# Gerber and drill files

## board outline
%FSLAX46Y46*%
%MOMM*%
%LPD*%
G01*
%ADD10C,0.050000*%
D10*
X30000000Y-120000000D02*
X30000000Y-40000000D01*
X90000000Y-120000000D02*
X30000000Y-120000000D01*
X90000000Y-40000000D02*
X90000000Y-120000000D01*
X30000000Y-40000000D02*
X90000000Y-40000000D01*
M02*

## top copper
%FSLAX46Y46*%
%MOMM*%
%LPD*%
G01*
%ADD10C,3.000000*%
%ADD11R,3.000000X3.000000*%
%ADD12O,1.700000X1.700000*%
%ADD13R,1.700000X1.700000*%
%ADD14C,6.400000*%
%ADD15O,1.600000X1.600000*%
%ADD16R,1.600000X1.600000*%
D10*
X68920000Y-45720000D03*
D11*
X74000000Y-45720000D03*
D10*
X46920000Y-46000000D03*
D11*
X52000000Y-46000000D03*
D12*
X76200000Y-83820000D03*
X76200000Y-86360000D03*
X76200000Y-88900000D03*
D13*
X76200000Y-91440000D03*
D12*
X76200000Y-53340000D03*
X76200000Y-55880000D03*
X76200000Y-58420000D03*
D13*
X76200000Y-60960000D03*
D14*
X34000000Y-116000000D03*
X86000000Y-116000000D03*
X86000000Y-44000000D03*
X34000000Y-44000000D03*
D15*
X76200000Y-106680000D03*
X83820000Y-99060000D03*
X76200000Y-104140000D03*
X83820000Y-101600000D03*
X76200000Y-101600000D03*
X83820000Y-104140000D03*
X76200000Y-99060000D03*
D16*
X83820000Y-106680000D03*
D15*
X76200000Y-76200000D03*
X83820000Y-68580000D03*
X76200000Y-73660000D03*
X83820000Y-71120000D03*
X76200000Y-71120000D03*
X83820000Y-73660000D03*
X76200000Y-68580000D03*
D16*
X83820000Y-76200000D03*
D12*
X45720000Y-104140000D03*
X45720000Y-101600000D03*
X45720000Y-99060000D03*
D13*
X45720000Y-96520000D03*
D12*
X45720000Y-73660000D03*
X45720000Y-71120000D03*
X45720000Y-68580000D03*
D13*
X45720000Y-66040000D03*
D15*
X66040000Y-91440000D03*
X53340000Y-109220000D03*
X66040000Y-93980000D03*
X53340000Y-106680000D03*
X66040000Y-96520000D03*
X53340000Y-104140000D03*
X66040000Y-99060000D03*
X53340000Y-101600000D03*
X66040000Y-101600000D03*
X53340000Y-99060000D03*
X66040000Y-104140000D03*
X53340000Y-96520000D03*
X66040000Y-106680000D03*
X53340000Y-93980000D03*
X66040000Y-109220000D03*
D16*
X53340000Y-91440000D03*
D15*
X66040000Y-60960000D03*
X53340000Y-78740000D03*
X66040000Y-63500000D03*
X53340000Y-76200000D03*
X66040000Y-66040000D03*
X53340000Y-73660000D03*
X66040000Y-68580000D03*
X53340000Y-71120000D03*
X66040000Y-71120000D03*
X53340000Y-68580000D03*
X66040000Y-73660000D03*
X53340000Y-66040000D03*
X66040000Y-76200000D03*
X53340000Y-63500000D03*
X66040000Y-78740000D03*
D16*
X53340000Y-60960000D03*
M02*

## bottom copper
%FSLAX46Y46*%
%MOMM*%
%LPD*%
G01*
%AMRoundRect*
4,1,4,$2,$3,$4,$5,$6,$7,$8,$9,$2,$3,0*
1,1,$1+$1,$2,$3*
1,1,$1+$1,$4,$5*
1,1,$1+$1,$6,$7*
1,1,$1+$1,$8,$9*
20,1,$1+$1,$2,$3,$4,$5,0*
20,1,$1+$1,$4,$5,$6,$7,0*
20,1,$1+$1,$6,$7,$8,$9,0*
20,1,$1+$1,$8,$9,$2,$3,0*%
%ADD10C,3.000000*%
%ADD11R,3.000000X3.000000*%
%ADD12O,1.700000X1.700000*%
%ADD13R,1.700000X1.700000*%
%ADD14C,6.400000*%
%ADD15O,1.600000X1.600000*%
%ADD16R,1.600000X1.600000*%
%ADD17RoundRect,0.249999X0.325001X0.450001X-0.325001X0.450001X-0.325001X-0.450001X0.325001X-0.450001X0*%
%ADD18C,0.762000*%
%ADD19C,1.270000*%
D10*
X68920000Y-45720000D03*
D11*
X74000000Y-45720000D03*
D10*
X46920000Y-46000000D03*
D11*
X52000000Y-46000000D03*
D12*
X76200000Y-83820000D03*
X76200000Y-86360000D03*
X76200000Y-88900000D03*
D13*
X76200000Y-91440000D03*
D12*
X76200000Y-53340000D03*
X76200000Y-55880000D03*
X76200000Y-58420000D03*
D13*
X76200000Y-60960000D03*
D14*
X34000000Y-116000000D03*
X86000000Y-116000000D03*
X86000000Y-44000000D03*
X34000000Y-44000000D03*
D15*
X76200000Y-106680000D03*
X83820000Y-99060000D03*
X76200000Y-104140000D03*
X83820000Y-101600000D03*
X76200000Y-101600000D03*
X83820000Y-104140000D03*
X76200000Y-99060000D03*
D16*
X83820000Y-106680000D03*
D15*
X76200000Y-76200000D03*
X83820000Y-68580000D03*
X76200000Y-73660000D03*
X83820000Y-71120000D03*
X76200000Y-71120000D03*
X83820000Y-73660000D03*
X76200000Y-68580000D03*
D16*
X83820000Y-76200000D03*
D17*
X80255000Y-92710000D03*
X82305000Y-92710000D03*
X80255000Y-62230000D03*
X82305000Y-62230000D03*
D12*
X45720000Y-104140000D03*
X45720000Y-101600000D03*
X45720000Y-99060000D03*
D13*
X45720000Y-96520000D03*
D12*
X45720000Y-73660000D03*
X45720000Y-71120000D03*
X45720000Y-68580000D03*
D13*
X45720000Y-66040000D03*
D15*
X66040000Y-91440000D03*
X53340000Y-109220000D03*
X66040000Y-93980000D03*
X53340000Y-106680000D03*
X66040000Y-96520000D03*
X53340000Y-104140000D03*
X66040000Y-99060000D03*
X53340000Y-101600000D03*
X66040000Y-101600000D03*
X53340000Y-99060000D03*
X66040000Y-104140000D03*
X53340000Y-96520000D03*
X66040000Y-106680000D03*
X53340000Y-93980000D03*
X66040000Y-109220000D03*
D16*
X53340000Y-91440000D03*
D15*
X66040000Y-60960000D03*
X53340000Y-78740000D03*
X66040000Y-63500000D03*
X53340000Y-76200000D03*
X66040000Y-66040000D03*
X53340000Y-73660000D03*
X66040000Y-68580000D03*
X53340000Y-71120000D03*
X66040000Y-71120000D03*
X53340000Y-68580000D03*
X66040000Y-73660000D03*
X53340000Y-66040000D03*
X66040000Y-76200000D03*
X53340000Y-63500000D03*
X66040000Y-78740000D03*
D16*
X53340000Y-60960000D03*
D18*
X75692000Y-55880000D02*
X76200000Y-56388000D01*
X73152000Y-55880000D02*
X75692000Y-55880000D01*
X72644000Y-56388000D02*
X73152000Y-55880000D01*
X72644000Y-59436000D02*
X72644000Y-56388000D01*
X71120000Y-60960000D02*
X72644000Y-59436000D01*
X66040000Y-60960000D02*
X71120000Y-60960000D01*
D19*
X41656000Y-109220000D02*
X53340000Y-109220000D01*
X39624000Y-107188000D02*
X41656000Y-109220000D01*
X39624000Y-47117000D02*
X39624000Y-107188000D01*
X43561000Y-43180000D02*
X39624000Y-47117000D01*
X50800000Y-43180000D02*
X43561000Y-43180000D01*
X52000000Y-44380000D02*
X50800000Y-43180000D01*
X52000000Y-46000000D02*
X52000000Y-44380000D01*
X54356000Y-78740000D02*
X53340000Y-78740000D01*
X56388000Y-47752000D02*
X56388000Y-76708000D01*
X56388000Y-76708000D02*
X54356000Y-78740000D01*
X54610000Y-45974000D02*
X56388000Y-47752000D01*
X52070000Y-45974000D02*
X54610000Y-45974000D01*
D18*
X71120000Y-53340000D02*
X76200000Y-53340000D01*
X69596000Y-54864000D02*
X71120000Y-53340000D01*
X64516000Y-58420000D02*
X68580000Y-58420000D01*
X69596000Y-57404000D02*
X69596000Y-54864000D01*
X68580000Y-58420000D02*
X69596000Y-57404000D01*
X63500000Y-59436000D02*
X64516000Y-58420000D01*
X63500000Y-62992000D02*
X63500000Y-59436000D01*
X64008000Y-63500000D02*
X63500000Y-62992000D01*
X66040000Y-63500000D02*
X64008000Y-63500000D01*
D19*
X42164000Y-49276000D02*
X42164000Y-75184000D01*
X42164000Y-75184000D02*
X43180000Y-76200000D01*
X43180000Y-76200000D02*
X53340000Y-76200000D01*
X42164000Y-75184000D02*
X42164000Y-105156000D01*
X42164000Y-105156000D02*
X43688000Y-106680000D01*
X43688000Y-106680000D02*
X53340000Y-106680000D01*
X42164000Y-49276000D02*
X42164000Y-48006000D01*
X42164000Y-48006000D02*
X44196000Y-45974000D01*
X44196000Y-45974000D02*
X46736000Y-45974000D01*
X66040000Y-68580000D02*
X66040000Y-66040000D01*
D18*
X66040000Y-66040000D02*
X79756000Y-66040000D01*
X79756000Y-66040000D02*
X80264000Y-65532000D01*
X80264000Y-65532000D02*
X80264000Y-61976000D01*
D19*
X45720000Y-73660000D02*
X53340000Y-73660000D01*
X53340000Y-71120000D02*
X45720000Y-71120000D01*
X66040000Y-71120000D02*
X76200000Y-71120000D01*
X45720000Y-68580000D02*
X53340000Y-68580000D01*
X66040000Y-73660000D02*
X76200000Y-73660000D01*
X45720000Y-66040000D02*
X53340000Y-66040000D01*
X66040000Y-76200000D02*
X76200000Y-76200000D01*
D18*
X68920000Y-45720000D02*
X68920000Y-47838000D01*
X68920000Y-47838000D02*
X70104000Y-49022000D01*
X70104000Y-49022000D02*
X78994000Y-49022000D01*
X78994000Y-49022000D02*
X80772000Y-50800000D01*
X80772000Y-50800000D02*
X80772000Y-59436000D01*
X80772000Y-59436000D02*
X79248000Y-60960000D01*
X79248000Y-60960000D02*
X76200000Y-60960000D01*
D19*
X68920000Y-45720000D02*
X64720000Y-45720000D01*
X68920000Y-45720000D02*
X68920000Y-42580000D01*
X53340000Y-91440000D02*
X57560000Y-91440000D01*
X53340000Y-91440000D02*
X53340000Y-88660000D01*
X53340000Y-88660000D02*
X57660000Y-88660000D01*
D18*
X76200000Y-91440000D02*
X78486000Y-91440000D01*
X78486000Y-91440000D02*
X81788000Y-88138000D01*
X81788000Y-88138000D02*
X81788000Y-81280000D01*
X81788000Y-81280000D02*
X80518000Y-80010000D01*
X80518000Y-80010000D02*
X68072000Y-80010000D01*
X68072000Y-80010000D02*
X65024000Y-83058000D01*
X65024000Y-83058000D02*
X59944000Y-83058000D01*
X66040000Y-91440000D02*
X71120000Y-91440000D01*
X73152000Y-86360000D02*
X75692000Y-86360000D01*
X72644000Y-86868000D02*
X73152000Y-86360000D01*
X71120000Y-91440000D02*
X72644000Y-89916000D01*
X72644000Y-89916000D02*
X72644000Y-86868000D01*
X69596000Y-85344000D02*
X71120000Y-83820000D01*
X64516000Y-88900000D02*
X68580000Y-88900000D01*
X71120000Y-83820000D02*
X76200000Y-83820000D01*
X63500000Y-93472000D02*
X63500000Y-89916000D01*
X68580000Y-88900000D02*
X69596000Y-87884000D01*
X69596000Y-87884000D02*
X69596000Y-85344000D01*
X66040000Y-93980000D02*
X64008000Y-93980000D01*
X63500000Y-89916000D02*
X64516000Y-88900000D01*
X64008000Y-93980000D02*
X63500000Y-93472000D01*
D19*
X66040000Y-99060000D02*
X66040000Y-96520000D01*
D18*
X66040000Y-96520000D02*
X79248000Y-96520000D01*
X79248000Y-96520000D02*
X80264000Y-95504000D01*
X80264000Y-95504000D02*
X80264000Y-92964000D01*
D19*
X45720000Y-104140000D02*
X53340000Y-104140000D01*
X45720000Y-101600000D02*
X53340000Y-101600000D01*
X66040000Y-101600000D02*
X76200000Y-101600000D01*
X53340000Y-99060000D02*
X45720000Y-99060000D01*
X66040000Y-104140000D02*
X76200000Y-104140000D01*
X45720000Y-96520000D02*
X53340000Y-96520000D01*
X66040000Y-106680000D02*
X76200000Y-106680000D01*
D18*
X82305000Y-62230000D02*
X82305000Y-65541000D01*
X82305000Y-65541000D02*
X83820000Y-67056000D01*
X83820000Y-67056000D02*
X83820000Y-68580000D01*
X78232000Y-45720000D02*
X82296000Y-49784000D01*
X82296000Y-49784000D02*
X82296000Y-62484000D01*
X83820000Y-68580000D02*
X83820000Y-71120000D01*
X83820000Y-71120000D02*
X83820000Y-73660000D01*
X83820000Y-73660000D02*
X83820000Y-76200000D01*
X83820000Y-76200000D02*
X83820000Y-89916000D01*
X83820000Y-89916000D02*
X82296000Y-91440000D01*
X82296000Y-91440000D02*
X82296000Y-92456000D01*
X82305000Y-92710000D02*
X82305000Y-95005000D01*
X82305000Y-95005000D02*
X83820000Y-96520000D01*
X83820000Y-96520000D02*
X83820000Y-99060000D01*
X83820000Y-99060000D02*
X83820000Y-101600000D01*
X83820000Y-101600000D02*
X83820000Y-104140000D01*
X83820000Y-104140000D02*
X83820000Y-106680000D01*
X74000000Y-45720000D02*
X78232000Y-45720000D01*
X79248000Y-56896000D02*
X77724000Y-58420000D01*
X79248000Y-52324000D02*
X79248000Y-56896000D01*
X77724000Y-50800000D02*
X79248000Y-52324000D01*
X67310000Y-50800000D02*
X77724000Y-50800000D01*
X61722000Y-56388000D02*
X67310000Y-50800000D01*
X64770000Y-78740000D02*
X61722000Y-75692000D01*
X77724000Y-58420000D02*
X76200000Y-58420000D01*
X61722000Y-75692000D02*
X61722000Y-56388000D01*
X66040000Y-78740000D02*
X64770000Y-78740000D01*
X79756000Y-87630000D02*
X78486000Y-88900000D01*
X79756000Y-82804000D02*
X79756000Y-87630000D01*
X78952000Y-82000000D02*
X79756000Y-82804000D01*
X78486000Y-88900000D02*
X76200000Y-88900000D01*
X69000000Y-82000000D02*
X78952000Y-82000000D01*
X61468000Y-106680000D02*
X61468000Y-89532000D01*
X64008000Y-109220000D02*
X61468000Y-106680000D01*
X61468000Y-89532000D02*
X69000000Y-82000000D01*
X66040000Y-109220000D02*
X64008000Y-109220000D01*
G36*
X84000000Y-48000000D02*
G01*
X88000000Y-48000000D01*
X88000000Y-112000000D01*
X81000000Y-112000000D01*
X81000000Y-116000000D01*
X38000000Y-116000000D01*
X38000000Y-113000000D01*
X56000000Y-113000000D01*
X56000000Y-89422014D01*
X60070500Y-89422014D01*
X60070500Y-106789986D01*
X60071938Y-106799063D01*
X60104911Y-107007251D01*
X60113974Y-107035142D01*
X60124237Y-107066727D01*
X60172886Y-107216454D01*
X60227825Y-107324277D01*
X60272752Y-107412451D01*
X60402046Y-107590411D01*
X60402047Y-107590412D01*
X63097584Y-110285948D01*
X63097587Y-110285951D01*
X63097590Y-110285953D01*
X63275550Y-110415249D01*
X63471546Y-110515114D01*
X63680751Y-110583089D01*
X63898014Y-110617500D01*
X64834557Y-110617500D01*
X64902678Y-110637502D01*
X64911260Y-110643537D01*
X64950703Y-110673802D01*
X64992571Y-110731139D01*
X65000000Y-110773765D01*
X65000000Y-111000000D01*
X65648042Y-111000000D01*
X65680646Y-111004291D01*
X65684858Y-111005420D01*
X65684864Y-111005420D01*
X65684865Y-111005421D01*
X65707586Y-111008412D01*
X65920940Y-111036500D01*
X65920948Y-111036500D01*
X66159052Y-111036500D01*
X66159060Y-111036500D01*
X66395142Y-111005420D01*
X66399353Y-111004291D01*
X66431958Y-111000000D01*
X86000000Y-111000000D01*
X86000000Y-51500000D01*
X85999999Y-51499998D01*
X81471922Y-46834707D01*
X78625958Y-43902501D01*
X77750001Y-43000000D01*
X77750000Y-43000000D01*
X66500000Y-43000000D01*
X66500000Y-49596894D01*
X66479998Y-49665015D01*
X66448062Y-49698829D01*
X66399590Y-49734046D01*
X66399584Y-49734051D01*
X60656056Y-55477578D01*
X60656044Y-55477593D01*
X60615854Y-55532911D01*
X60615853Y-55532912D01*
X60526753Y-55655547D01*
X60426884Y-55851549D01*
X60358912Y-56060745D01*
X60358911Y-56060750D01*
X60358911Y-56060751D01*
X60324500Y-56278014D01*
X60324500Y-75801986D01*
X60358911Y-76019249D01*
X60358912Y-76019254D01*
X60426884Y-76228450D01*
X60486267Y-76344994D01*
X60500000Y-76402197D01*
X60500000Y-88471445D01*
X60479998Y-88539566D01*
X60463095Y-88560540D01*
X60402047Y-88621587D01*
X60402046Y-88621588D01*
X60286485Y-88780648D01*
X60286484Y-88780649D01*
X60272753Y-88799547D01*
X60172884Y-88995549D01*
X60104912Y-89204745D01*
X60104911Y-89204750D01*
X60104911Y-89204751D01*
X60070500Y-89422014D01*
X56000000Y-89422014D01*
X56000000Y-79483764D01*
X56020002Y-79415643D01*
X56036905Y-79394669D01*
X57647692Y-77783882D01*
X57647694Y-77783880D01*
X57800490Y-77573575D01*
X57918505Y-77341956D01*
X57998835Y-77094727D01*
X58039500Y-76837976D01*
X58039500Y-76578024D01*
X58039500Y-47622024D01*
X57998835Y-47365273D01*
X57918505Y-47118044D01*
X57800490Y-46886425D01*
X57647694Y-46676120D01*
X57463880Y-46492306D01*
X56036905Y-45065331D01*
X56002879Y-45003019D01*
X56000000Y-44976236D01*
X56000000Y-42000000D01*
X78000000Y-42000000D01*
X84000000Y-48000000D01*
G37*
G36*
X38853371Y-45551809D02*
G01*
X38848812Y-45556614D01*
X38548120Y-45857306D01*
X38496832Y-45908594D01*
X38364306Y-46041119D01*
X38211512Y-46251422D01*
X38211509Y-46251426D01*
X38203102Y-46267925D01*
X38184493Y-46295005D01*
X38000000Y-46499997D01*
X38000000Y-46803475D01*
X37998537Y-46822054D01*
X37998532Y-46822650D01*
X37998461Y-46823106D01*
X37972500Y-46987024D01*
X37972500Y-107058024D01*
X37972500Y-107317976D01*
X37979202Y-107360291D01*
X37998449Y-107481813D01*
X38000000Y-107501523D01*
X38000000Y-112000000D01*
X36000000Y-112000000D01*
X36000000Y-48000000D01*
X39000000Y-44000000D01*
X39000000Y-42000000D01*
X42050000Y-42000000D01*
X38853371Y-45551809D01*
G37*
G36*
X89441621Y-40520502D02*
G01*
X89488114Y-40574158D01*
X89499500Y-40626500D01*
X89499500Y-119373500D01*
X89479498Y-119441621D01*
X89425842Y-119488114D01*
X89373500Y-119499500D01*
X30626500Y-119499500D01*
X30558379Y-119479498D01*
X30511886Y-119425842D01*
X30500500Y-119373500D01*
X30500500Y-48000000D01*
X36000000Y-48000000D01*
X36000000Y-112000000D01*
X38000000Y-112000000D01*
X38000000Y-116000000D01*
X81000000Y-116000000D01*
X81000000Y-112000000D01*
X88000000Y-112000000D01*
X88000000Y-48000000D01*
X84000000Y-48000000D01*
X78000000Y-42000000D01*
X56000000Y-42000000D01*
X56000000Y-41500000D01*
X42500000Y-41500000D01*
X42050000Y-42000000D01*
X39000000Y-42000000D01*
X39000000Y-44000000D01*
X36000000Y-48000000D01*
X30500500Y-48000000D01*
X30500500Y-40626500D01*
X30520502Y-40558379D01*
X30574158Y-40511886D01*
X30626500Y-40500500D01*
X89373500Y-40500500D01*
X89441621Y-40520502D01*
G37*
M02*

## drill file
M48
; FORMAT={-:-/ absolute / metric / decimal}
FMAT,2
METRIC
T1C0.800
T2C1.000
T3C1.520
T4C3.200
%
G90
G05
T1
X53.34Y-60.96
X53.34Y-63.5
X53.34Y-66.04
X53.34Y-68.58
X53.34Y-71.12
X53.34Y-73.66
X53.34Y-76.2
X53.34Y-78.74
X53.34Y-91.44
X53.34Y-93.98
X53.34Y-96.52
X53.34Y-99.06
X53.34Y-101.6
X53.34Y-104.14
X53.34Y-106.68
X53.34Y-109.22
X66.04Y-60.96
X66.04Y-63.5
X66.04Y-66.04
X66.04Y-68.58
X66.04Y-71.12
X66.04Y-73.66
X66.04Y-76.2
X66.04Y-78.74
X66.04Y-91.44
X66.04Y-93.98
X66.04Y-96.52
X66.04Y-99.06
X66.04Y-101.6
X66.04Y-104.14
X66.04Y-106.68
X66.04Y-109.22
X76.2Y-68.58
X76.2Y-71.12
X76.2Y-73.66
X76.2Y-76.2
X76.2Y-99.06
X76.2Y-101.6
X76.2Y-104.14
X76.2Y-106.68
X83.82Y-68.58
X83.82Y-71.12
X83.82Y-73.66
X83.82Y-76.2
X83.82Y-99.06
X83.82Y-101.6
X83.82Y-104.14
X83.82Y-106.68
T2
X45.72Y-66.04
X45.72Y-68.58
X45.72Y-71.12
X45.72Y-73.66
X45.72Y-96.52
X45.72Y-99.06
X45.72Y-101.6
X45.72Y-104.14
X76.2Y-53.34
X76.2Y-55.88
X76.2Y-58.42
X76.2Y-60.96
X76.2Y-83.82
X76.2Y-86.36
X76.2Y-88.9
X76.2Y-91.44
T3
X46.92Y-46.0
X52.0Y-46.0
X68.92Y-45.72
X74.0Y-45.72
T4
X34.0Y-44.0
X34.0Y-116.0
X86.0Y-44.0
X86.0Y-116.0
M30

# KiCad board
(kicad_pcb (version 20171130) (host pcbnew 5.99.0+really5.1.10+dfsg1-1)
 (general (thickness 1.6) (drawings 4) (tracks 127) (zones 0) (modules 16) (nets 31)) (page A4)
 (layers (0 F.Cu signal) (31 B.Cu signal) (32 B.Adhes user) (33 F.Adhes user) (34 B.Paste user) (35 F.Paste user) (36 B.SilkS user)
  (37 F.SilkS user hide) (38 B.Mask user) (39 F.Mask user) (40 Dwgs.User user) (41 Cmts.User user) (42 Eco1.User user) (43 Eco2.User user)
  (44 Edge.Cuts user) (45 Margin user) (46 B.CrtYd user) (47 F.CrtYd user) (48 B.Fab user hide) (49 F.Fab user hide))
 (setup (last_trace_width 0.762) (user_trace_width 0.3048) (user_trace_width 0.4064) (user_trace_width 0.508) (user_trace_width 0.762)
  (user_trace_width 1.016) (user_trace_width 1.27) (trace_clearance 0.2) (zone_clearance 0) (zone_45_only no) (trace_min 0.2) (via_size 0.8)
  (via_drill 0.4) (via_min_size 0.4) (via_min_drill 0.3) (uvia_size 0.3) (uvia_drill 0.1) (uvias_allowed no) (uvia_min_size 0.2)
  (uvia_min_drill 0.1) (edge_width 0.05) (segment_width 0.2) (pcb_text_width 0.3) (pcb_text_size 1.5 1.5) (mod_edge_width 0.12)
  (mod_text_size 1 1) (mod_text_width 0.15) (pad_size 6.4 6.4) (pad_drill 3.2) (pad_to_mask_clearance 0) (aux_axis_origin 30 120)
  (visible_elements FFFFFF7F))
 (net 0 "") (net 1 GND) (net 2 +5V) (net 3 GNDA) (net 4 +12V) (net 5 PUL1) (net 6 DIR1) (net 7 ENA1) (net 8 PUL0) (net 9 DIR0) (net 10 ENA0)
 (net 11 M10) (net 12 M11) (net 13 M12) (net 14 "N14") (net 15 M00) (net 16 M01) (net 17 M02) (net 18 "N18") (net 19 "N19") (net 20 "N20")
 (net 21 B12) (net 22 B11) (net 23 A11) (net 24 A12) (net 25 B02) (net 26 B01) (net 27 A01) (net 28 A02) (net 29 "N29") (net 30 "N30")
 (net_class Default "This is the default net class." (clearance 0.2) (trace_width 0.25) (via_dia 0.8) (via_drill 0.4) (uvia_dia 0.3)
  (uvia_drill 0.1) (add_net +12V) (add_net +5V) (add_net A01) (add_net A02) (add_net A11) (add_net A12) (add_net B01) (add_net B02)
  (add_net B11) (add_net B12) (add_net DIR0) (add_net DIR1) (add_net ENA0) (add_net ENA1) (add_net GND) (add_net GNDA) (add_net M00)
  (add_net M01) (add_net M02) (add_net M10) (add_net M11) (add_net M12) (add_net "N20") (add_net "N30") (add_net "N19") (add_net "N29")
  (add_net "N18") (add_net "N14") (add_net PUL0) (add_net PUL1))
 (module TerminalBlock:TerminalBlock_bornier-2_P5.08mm (layer F.Cu) (at 74 45.72 180)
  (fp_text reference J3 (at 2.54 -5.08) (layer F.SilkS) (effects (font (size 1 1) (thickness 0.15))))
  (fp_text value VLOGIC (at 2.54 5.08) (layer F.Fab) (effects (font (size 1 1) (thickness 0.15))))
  (pad 2 thru_hole circle (at 5.08 0 180) (size 3 3) (drill 1.52) (layers *.Cu *.Mask) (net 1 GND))
  (pad 1 thru_hole rect (at 0 0 180) (size 3 3) (drill 1.52) (layers *.Cu *.Mask) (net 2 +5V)))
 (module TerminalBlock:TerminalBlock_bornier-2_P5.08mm (layer F.Cu) (at 52 46 180)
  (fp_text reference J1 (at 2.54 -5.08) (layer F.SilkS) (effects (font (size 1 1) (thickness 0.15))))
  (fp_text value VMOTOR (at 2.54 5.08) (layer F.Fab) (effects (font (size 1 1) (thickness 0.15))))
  (pad 2 thru_hole circle (at 5.08 0 180) (size 3 3) (drill 1.52) (layers *.Cu *.Mask) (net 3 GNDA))
  (pad 1 thru_hole rect (at 0 0 180) (size 3 3) (drill 1.52) (layers *.Cu *.Mask) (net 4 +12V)))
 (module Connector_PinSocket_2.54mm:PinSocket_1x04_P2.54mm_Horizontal (layer F.Cu) (at 76.2 91.44 180)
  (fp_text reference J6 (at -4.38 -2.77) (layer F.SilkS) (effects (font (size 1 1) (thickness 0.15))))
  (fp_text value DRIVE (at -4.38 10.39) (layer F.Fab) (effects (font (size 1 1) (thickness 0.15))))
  (pad 4 thru_hole oval (at 0 7.62 180) (size 1.7 1.7) (drill 1) (layers *.Cu *.Mask) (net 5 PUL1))
  (pad 3 thru_hole oval (at 0 5.08 180) (size 1.7 1.7) (drill 1) (layers *.Cu *.Mask) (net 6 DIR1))
  (pad 2 thru_hole oval (at 0 2.54 180) (size 1.7 1.7) (drill 1) (layers *.Cu *.Mask) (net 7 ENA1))
  (pad 1 thru_hole rect (at 0 0 180) (size 1.7 1.7) (drill 1) (layers *.Cu *.Mask) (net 1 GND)))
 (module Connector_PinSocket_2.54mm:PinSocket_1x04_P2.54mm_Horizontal (layer F.Cu) (at 76.2 60.96 180)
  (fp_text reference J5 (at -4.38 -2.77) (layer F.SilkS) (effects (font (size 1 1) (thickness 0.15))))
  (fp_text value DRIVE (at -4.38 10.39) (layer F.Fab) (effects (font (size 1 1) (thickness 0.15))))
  (pad 4 thru_hole oval (at 0 7.62 180) (size 1.7 1.7) (drill 1) (layers *.Cu *.Mask) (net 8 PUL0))
  (pad 3 thru_hole oval (at 0 5.08 180) (size 1.7 1.7) (drill 1) (layers *.Cu *.Mask) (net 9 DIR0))
  (pad 2 thru_hole oval (at 0 2.54 180) (size 1.7 1.7) (drill 1) (layers *.Cu *.Mask) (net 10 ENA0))
  (pad 1 thru_hole rect (at 0 0 180) (size 1.7 1.7) (drill 1) (layers *.Cu *.Mask) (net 1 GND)))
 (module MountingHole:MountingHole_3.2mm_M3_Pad (layer F.Cu) (at 34 116)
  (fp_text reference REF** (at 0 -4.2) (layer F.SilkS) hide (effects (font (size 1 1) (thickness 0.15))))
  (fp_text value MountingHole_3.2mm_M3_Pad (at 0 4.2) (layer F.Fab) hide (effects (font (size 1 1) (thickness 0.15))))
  (pad 1 thru_hole circle (at 0 0) (size 6.4 6.4) (drill 3.2) (layers *.Cu *.Mask) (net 1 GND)))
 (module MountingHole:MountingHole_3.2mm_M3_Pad (layer F.Cu) (at 86 116)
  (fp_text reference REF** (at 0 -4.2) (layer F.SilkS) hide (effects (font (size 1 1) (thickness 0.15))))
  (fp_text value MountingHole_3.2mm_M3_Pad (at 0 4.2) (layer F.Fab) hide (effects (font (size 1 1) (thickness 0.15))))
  (pad 1 thru_hole circle (at 0 0) (size 6.4 6.4) (drill 3.2) (layers *.Cu *.Mask) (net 1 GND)))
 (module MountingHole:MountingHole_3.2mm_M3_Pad (layer F.Cu) (at 86 44)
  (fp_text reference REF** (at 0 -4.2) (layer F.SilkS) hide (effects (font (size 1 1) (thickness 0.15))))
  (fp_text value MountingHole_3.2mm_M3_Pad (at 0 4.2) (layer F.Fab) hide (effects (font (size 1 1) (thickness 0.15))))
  (pad 1 thru_hole circle (at 0 0) (size 6.4 6.4) (drill 3.2) (layers *.Cu *.Mask) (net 1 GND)))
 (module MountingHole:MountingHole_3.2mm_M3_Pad (layer F.Cu) (at 34 44)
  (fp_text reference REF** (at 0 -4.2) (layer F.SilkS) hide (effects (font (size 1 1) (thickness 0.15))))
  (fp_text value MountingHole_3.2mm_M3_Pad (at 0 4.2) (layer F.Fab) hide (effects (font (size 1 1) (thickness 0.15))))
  (pad 1 thru_hole circle (at 0 0) (size 6.4 6.4) (drill 3.2) (layers *.Cu *.Mask) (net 1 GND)))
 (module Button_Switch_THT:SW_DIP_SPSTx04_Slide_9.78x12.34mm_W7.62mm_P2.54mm (layer F.Cu) (at 83.82 106.68 180)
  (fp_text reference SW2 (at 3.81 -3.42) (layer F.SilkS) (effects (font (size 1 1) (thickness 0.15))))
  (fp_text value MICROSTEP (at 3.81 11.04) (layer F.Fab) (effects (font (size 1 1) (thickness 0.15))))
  (pad 8 thru_hole oval (at 7.62 0 180) (size 1.6 1.6) (drill 0.8) (layers *.Cu *.Mask) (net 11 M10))
  (pad 4 thru_hole oval (at 0 7.62 180) (size 1.6 1.6) (drill 0.8) (layers *.Cu *.Mask) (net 2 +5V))
  (pad 7 thru_hole oval (at 7.62 2.54 180) (size 1.6 1.6) (drill 0.8) (layers *.Cu *.Mask) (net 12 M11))
  (pad 3 thru_hole oval (at 0 5.08 180) (size 1.6 1.6) (drill 0.8) (layers *.Cu *.Mask) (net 2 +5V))
  (pad 6 thru_hole oval (at 7.62 5.08 180) (size 1.6 1.6) (drill 0.8) (layers *.Cu *.Mask) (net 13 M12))
  (pad 2 thru_hole oval (at 0 2.54 180) (size 1.6 1.6) (drill 0.8) (layers *.Cu *.Mask) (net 2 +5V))
  (pad 5 thru_hole oval (at 7.62 7.62 180) (size 1.6 1.6) (drill 0.8) (layers *.Cu *.Mask) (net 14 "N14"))
  (pad 1 thru_hole rect (at 0 0 180) (size 1.6 1.6) (drill 0.8) (layers *.Cu *.Mask) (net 2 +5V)))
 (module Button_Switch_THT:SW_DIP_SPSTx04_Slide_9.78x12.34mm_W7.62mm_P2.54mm (layer F.Cu) (at 83.82 76.2 180)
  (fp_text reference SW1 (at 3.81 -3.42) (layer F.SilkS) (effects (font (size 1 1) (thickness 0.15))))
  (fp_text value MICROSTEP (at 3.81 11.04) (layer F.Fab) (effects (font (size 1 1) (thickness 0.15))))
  (pad 8 thru_hole oval (at 7.62 0 180) (size 1.6 1.6) (drill 0.8) (layers *.Cu *.Mask) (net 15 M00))
  (pad 4 thru_hole oval (at 0 7.62 180) (size 1.6 1.6) (drill 0.8) (layers *.Cu *.Mask) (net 2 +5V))
  (pad 7 thru_hole oval (at 7.62 2.54 180) (size 1.6 1.6) (drill 0.8) (layers *.Cu *.Mask) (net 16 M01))
  (pad 3 thru_hole oval (at 0 5.08 180) (size 1.6 1.6) (drill 0.8) (layers *.Cu *.Mask) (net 2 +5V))
  (pad 6 thru_hole oval (at 7.62 5.08 180) (size 1.6 1.6) (drill 0.8) (layers *.Cu *.Mask) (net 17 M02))
  (pad 2 thru_hole oval (at 0 2.54 180) (size 1.6 1.6) (drill 0.8) (layers *.Cu *.Mask) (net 2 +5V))
  (pad 5 thru_hole oval (at 7.62 7.62 180) (size 1.6 1.6) (drill 0.8) (layers *.Cu *.Mask) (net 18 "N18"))
  (pad 1 thru_hole rect (at 0 0 180) (size 1.6 1.6) (drill 0.8) (layers *.Cu *.Mask) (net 2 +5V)))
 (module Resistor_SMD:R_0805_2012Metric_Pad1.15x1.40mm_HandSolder (layer B.Cu) (at 81.28 92.71 180)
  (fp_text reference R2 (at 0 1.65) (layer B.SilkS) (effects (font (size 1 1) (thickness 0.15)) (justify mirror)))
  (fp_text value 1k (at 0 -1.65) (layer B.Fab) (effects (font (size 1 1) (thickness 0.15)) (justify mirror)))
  (pad 2 smd roundrect (at 1.025 0 180) (size 1.15 1.4) (layers B.Cu B.Paste B.Mask) (roundrect_rratio 0.2173904347826087) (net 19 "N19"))
  (pad 1 smd roundrect (at -1.025 0 180) (size 1.15 1.4) (layers B.Cu B.Paste B.Mask) (roundrect_rratio 0.2173904347826087) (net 2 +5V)))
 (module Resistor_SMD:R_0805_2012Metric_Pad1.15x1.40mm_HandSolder (layer B.Cu) (at 81.28 62.23 180)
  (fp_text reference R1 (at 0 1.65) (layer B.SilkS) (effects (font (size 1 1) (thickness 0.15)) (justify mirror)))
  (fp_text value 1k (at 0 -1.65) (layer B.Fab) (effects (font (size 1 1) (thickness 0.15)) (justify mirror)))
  (pad 2 smd roundrect (at 1.025 0 180) (size 1.15 1.4) (layers B.Cu B.Paste B.Mask) (roundrect_rratio 0.2173904347826087) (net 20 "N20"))
  (pad 1 smd roundrect (at -1.025 0 180) (size 1.15 1.4) (layers B.Cu B.Paste B.Mask) (roundrect_rratio 0.2173904347826087) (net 2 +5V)))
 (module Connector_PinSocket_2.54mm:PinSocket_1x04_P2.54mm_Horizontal (layer F.Cu) (at 45.72 96.52)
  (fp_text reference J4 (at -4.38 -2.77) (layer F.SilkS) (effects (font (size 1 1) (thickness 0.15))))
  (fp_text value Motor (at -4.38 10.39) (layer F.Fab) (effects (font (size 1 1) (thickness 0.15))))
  (pad 4 thru_hole oval (at 0 7.62) (size 1.7 1.7) (drill 1) (layers *.Cu *.Mask) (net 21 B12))
  (pad 3 thru_hole oval (at 0 5.08) (size 1.7 1.7) (drill 1) (layers *.Cu *.Mask) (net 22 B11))
  (pad 2 thru_hole oval (at 0 2.54) (size 1.7 1.7) (drill 1) (layers *.Cu *.Mask) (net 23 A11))
  (pad 1 thru_hole rect (at 0 0) (size 1.7 1.7) (drill 1) (layers *.Cu *.Mask) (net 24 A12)))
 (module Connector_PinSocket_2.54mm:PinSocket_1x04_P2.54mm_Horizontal (layer F.Cu) (at 45.72 66.04)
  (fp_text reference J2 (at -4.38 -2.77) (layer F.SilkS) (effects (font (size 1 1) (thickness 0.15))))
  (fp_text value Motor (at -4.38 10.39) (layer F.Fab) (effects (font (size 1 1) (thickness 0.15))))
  (pad 4 thru_hole oval (at 0 7.62) (size 1.7 1.7) (drill 1) (layers *.Cu *.Mask) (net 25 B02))
  (pad 3 thru_hole oval (at 0 5.08) (size 1.7 1.7) (drill 1) (layers *.Cu *.Mask) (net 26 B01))
  (pad 2 thru_hole oval (at 0 2.54) (size 1.7 1.7) (drill 1) (layers *.Cu *.Mask) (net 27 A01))
  (pad 1 thru_hole rect (at 0 0) (size 1.7 1.7) (drill 1) (layers *.Cu *.Mask) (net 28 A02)))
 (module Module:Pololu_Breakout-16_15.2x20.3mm (layer F.Cu) (at 53.34 91.44)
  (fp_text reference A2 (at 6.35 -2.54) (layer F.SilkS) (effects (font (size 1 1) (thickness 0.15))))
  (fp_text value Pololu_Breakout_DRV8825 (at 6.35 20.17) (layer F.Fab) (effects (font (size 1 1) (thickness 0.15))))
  (pad 16 thru_hole oval (at 12.7 0) (size 1.6 1.6) (drill 0.8) (layers *.Cu *.Mask) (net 6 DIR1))
  (pad 8 thru_hole oval (at 0 17.78) (size 1.6 1.6) (drill 0.8) (layers *.Cu *.Mask) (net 4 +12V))
  (pad 15 thru_hole oval (at 12.7 2.54) (size 1.6 1.6) (drill 0.8) (layers *.Cu *.Mask) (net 5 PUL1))
  (pad 7 thru_hole oval (at 0 15.24) (size 1.6 1.6) (drill 0.8) (layers *.Cu *.Mask) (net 3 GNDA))
  (pad 14 thru_hole oval (at 12.7 5.08) (size 1.6 1.6) (drill 0.8) (layers *.Cu *.Mask) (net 19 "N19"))
  (pad 6 thru_hole oval (at 0 12.7) (size 1.6 1.6) (drill 0.8) (layers *.Cu *.Mask) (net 21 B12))
  (pad 13 thru_hole oval (at 12.7 7.62) (size 1.6 1.6) (drill 0.8) (layers *.Cu *.Mask) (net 19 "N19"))
  (pad 5 thru_hole oval (at 0 10.16) (size 1.6 1.6) (drill 0.8) (layers *.Cu *.Mask) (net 22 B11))
  (pad 12 thru_hole oval (at 12.7 10.16) (size 1.6 1.6) (drill 0.8) (layers *.Cu *.Mask) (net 13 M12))
  (pad 4 thru_hole oval (at 0 7.62) (size 1.6 1.6) (drill 0.8) (layers *.Cu *.Mask) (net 23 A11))
  (pad 11 thru_hole oval (at 12.7 12.7) (size 1.6 1.6) (drill 0.8) (layers *.Cu *.Mask) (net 12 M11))
  (pad 3 thru_hole oval (at 0 5.08) (size 1.6 1.6) (drill 0.8) (layers *.Cu *.Mask) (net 24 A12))
  (pad 10 thru_hole oval (at 12.7 15.24) (size 1.6 1.6) (drill 0.8) (layers *.Cu *.Mask) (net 11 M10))
  (pad 2 thru_hole oval (at 0 2.54) (size 1.6 1.6) (drill 0.8) (layers *.Cu *.Mask) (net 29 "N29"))
  (pad 9 thru_hole oval (at 12.7 17.78) (size 1.6 1.6) (drill 0.8) (layers *.Cu *.Mask) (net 7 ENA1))
  (pad 1 thru_hole rect (at 0 0) (size 1.6 1.6) (drill 0.8) (layers *.Cu *.Mask) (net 1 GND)))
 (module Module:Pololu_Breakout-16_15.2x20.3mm (layer F.Cu) (at 53.34 60.96)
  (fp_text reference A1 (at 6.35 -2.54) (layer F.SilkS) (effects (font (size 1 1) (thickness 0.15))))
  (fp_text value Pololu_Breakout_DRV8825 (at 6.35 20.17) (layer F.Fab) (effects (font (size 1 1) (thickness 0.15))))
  (pad 16 thru_hole oval (at 12.7 0) (size 1.6 1.6) (drill 0.8) (layers *.Cu *.Mask) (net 9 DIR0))
  (pad 8 thru_hole oval (at 0 17.78) (size 1.6 1.6) (drill 0.8) (layers *.Cu *.Mask) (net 4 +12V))
  (pad 15 thru_hole oval (at 12.7 2.54) (size 1.6 1.6) (drill 0.8) (layers *.Cu *.Mask) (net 8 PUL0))
  (pad 7 thru_hole oval (at 0 15.24) (size 1.6 1.6) (drill 0.8) (layers *.Cu *.Mask) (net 3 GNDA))
  (pad 14 thru_hole oval (at 12.7 5.08) (size 1.6 1.6) (drill 0.8) (layers *.Cu *.Mask) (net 20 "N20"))
  (pad 6 thru_hole oval (at 0 12.7) (size 1.6 1.6) (drill 0.8) (layers *.Cu *.Mask) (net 25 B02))
  (pad 13 thru_hole oval (at 12.7 7.62) (size 1.6 1.6) (drill 0.8) (layers *.Cu *.Mask) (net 20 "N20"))
  (pad 5 thru_hole oval (at 0 10.16) (size 1.6 1.6) (drill 0.8) (layers *.Cu *.Mask) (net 26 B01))
  (pad 12 thru_hole oval (at 12.7 10.16) (size 1.6 1.6) (drill 0.8) (layers *.Cu *.Mask) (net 17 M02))
  (pad 4 thru_hole oval (at 0 7.62) (size 1.6 1.6) (drill 0.8) (layers *.Cu *.Mask) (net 27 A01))
  (pad 11 thru_hole oval (at 12.7 12.7) (size 1.6 1.6) (drill 0.8) (layers *.Cu *.Mask) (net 16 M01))
  (pad 3 thru_hole oval (at 0 5.08) (size 1.6 1.6) (drill 0.8) (layers *.Cu *.Mask) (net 28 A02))
  (pad 10 thru_hole oval (at 12.7 15.24) (size 1.6 1.6) (drill 0.8) (layers *.Cu *.Mask) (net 15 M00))
  (pad 2 thru_hole oval (at 0 2.54) (size 1.6 1.6) (drill 0.8) (layers *.Cu *.Mask) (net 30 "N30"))
  (pad 9 thru_hole oval (at 12.7 17.78) (size 1.6 1.6) (drill 0.8) (layers *.Cu *.Mask) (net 10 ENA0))
  (pad 1 thru_hole rect (at 0 0) (size 1.6 1.6) (drill 0.8) (layers *.Cu *.Mask) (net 1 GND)))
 (gr_line (start 30 120) (end 30 40) (layer Edge.Cuts) (width 0.05))
 (gr_line (start 90 120) (end 30 120) (layer Edge.Cuts) (width 0.05))
 (gr_line (start 90 40) (end 90 120) (layer Edge.Cuts) (width 0.05))
 (gr_line (start 30 40) (end 90 40) (layer Edge.Cuts) (width 0.05))
 (segment (start 75.692 55.88) (end 76.2 56.388) (width 0.762) (layer B.Cu) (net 9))
 (segment (start 73.152 55.88) (end 75.692 55.88) (width 0.762) (layer B.Cu) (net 9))
 (segment (start 72.644 56.388) (end 73.152 55.88) (width 0.762) (layer B.Cu) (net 9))
 (segment (start 72.644 59.436) (end 72.644 56.388) (width 0.762) (layer B.Cu) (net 9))
 (segment (start 71.12 60.96) (end 72.644 59.436) (width 0.762) (layer B.Cu) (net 9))
 (segment (start 66.04 60.96) (end 71.12 60.96) (width 0.762) (layer B.Cu) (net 9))
 (segment (start 41.656 109.22) (end 53.34 109.22) (width 1.27) (layer B.Cu) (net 4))
 (segment (start 39.624 107.188) (end 41.656 109.22) (width 1.27) (layer B.Cu) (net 4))
 (segment (start 39.624 47.117) (end 39.624 107.188) (width 1.27) (layer B.Cu) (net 4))
 (segment (start 43.561 43.18) (end 39.624 47.117) (width 1.27) (layer B.Cu) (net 4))
 (segment (start 50.8 43.18) (end 43.561 43.18) (width 1.27) (layer B.Cu) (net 4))
 (segment (start 52 44.38) (end 50.8 43.18) (width 1.27) (layer B.Cu) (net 4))
 (segment (start 52 46) (end 52 44.38) (width 1.27) (layer B.Cu) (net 4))
 (segment (start 54.356 78.74) (end 53.34 78.74) (width 1.27) (layer B.Cu) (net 4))
 (segment (start 56.388 47.752) (end 56.388 76.708) (width 1.27) (layer B.Cu) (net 4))
 (segment (start 56.388 76.708) (end 54.356 78.74) (width 1.27) (layer B.Cu) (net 4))
 (segment (start 54.61 45.974) (end 56.388 47.752) (width 1.27) (layer B.Cu) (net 4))
 (segment (start 52.07 45.974) (end 54.61 45.974) (width 1.27) (layer B.Cu) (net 4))
 (segment (start 71.12 53.34) (end 76.2 53.34) (width 0.762) (layer B.Cu) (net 8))
 (segment (start 69.596 54.864) (end 71.12 53.34) (width 0.762) (layer B.Cu) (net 8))
 (segment (start 64.516 58.42) (end 68.58 58.42) (width 0.762) (layer B.Cu) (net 8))
 (segment (start 69.596 57.404) (end 69.596 54.864) (width 0.762) (layer B.Cu) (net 8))
 (segment (start 68.58 58.42) (end 69.596 57.404) (width 0.762) (layer B.Cu) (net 8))
 (segment (start 63.5 59.436) (end 64.516 58.42) (width 0.762) (layer B.Cu) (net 8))
 (segment (start 63.5 62.992) (end 63.5 59.436) (width 0.762) (layer B.Cu) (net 8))
 (segment (start 64.008 63.5) (end 63.5 62.992) (width 0.762) (layer B.Cu) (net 8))
 (segment (start 66.04 63.5) (end 64.008 63.5) (width 0.762) (layer B.Cu) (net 8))
 (segment (start 42.164 49.276) (end 42.164 75.184) (width 1.27) (layer B.Cu) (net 3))
 (segment (start 42.164 75.184) (end 43.18 76.2) (width 1.27) (layer B.Cu) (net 3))
 (segment (start 43.18 76.2) (end 53.34 76.2) (width 1.27) (layer B.Cu) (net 3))
 (segment (start 42.164 75.184) (end 42.164 105.156) (width 1.27) (layer B.Cu) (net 3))
 (segment (start 42.164 105.156) (end 43.688 106.68) (width 1.27) (layer B.Cu) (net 3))
 (segment (start 43.688 106.68) (end 53.34 106.68) (width 1.27) (layer B.Cu) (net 3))
 (segment (start 42.164 49.276) (end 42.164 48.006) (width 1.27) (layer B.Cu) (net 3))
 (segment (start 42.164 48.006) (end 44.196 45.974) (width 1.27) (layer B.Cu) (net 3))
 (segment (start 44.196 45.974) (end 46.736 45.974) (width 1.27) (layer B.Cu) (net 3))
 (segment (start 66.04 68.58) (end 66.04 66.04) (width 1.27) (layer B.Cu) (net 20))
 (segment (start 66.04 66.04) (end 79.756 66.04) (width 0.762) (layer B.Cu) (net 20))
 (segment (start 79.756 66.04) (end 80.264 65.532) (width 0.762) (layer B.Cu) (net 20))
 (segment (start 80.264 65.532) (end 80.264 61.976) (width 0.762) (layer B.Cu) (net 20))
 (segment (start 45.72 73.66) (end 53.34 73.66) (width 1.27) (layer B.Cu) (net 25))
 (segment (start 53.34 71.12) (end 45.72 71.12) (width 1.27) (layer B.Cu) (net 26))
 (segment (start 66.04 71.12) (end 76.2 71.12) (width 1.27) (layer B.Cu) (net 17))
 (segment (start 45.72 68.58) (end 53.34 68.58) (width 1.27) (layer B.Cu) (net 27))
 (segment (start 66.04 73.66) (end 76.2 73.66) (width 1.27) (layer B.Cu) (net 16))
 (segment (start 45.72 66.04) (end 53.34 66.04) (width 1.27) (layer B.Cu) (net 28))
 (segment (start 66.04 76.2) (end 76.2 76.2) (width 1.27) (layer B.Cu) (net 15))
 (segment (start 68.92 45.72) (end 68.92 47.838) (width 0.762) (layer B.Cu) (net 1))
 (segment (start 68.92 47.838) (end 70.104 49.022) (width 0.762) (layer B.Cu) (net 1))
 (segment (start 70.104 49.022) (end 78.994 49.022) (width 0.762) (layer B.Cu) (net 1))
 (segment (start 78.994 49.022) (end 80.772 50.8) (width 0.762) (layer B.Cu) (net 1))
 (segment (start 80.772 50.8) (end 80.772 59.436) (width 0.762) (layer B.Cu) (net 1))
 (segment (start 80.772 59.436) (end 79.248 60.96) (width 0.762) (layer B.Cu) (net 1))
 (segment (start 79.248 60.96) (end 76.2 60.96) (width 0.762) (layer B.Cu) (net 1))
 (segment (start 68.92 45.72) (end 64.72 45.72) (width 1.27) (layer B.Cu) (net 1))
 (segment (start 68.92 45.72) (end 68.92 42.58) (width 1.27) (layer B.Cu) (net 1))
 (segment (start 53.34 91.44) (end 57.56 91.44) (width 1.27) (layer B.Cu) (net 1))
 (segment (start 53.34 91.44) (end 53.34 88.66) (width 1.27) (layer B.Cu) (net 1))
 (segment (start 53.34 88.66) (end 57.66 88.66) (width 1.27) (layer B.Cu) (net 1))
 (segment (start 76.2 91.44) (end 78.486 91.44) (width 0.762) (layer B.Cu) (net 1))
 (segment (start 78.486 91.44) (end 81.788 88.138) (width 0.762) (layer B.Cu) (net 1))
 (segment (start 81.788 88.138) (end 81.788 81.28) (width 0.762) (layer B.Cu) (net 1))
 (segment (start 81.788 81.28) (end 80.518 80.01) (width 0.762) (layer B.Cu) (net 1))
 (segment (start 80.518 80.01) (end 68.072 80.01) (width 0.762) (layer B.Cu) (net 1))
 (segment (start 68.072 80.01) (end 65.024 83.058) (width 0.762) (layer B.Cu) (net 1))
 (segment (start 65.024 83.058) (end 59.944 83.058) (width 0.762) (layer B.Cu) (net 1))
 (segment (start 66.04 91.44) (end 71.12 91.44) (width 0.762) (layer B.Cu) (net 6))
 (segment (start 73.152 86.36) (end 75.692 86.36) (width 0.762) (layer B.Cu) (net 6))
 (segment (start 72.644 86.868) (end 73.152 86.36) (width 0.762) (layer B.Cu) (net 6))
 (segment (start 71.12 91.44) (end 72.644 89.916) (width 0.762) (layer B.Cu) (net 6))
 (segment (start 72.644 89.916) (end 72.644 86.868) (width 0.762) (layer B.Cu) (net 6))
 (segment (start 69.596 85.344) (end 71.12 83.82) (width 0.762) (layer B.Cu) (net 5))
 (segment (start 64.516 88.9) (end 68.58 88.9) (width 0.762) (layer B.Cu) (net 5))
 (segment (start 71.12 83.82) (end 76.2 83.82) (width 0.762) (layer B.Cu) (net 5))
 (segment (start 63.5 93.472) (end 63.5 89.916) (width 0.762) (layer B.Cu) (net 5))
 (segment (start 68.58 88.9) (end 69.596 87.884) (width 0.762) (layer B.Cu) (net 5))
 (segment (start 69.596 87.884) (end 69.596 85.344) (width 0.762) (layer B.Cu) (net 5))
 (segment (start 66.04 93.98) (end 64.008 93.98) (width 0.762) (layer B.Cu) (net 5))
 (segment (start 63.5 89.916) (end 64.516 88.9) (width 0.762) (layer B.Cu) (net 5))
 (segment (start 64.008 93.98) (end 63.5 93.472) (width 0.762) (layer B.Cu) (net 5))
 (segment (start 66.04 99.06) (end 66.04 96.52) (width 1.27) (layer B.Cu) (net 19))
 (segment (start 66.04 96.52) (end 79.248 96.52) (width 0.762) (layer B.Cu) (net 19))
 (segment (start 79.248 96.52) (end 80.264 95.504) (width 0.762) (layer B.Cu) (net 19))
 (segment (start 80.264 95.504) (end 80.264 92.964) (width 0.762) (layer B.Cu) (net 19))
 (segment (start 45.72 104.14) (end 53.34 104.14) (width 1.27) (layer B.Cu) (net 21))
 (segment (start 45.72 101.6) (end 53.34 101.6) (width 1.27) (layer B.Cu) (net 22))
 (segment (start 66.04 101.6) (end 76.2 101.6) (width 1.27) (layer B.Cu) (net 13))
 (segment (start 53.34 99.06) (end 45.72 99.06) (width 1.27) (layer B.Cu) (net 23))
 (segment (start 66.04 104.14) (end 76.2 104.14) (width 1.27) (layer B.Cu) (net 12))
 (segment (start 45.72 96.52) (end 53.34 96.52) (width 1.27) (layer B.Cu) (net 24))
 (segment (start 66.04 106.68) (end 76.2 106.68) (width 1.27) (layer B.Cu) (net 11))
 (segment (start 82.305 62.23) (end 82.305 65.541) (width 0.762) (layer B.Cu) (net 2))
 (segment (start 82.305 65.541) (end 83.82 67.056) (width 0.762) (layer B.Cu) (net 2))
 (segment (start 83.82 67.056) (end 83.82 68.58) (width 0.762) (layer B.Cu) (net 2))
 (segment (start 78.232 45.72) (end 82.296 49.784) (width 0.762) (layer B.Cu) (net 2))
 (segment (start 82.296 49.784) (end 82.296 62.484) (width 0.762) (layer B.Cu) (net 2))
 (segment (start 83.82 68.58) (end 83.82 71.12) (width 0.762) (layer B.Cu) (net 2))
 (segment (start 83.82 71.12) (end 83.82 73.66) (width 0.762) (layer B.Cu) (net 2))
 (segment (start 83.82 73.66) (end 83.82 76.2) (width 0.762) (layer B.Cu) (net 2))
 (segment (start 83.82 76.2) (end 83.82 89.916) (width 0.762) (layer B.Cu) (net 2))
 (segment (start 83.82 89.916) (end 82.296 91.44) (width 0.762) (layer B.Cu) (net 2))
 (segment (start 82.296 91.44) (end 82.296 92.456) (width 0.762) (layer B.Cu) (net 2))
 (segment (start 82.305 92.71) (end 82.305 95.005) (width 0.762) (layer B.Cu) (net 2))
 (segment (start 82.305 95.005) (end 83.82 96.52) (width 0.762) (layer B.Cu) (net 2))
 (segment (start 83.82 96.52) (end 83.82 99.06) (width 0.762) (layer B.Cu) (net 2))
 (segment (start 83.82 99.06) (end 83.82 101.6) (width 0.762) (layer B.Cu) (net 2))
 (segment (start 83.82 101.6) (end 83.82 104.14) (width 0.762) (layer B.Cu) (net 2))
 (segment (start 83.82 104.14) (end 83.82 106.68) (width 0.762) (layer B.Cu) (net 2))
 (segment (start 74 45.72) (end 78.232 45.72) (width 0.762) (layer B.Cu) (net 2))
 (segment (start 79.248 56.896) (end 77.724 58.42) (width 0.762) (layer B.Cu) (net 10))
 (segment (start 79.248 52.324) (end 79.248 56.896) (width 0.762) (layer B.Cu) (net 10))
 (segment (start 77.724 50.8) (end 79.248 52.324) (width 0.762) (layer B.Cu) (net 10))
 (segment (start 67.31 50.8) (end 77.724 50.8) (width 0.762) (layer B.Cu) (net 10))
 (segment (start 61.722 56.388) (end 67.31 50.8) (width 0.762) (layer B.Cu) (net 10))
 (segment (start 64.77 78.74) (end 61.722 75.692) (width 0.762) (layer B.Cu) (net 10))
 (segment (start 77.724 58.42) (end 76.2 58.42) (width 0.762) (layer B.Cu) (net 10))
 (segment (start 61.722 75.692) (end 61.722 56.388) (width 0.762) (layer B.Cu) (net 10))
 (segment (start 66.04 78.74) (end 64.77 78.74) (width 0.762) (layer B.Cu) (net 10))
 (segment (start 79.756 87.63) (end 78.486 88.9) (width 0.762) (layer B.Cu) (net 7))
 (segment (start 79.756 82.804) (end 79.756 87.63) (width 0.762) (layer B.Cu) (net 7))
 (segment (start 78.952 82) (end 79.756 82.804) (width 0.762) (layer B.Cu) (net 7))
 (segment (start 78.486 88.9) (end 76.2 88.9) (width 0.762) (layer B.Cu) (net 7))
 (segment (start 69 82) (end 78.952 82) (width 0.762) (layer B.Cu) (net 7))
 (segment (start 61.468 106.68) (end 61.468 89.532) (width 0.762) (layer B.Cu) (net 7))
 (segment (start 64.008 109.22) (end 61.468 106.68) (width 0.762) (layer B.Cu) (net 7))
 (segment (start 61.468 89.532) (end 69 82) (width 0.762) (layer B.Cu) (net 7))
 (segment (start 66.04 109.22) (end 64.008 109.22) (width 0.762) (layer B.Cu) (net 7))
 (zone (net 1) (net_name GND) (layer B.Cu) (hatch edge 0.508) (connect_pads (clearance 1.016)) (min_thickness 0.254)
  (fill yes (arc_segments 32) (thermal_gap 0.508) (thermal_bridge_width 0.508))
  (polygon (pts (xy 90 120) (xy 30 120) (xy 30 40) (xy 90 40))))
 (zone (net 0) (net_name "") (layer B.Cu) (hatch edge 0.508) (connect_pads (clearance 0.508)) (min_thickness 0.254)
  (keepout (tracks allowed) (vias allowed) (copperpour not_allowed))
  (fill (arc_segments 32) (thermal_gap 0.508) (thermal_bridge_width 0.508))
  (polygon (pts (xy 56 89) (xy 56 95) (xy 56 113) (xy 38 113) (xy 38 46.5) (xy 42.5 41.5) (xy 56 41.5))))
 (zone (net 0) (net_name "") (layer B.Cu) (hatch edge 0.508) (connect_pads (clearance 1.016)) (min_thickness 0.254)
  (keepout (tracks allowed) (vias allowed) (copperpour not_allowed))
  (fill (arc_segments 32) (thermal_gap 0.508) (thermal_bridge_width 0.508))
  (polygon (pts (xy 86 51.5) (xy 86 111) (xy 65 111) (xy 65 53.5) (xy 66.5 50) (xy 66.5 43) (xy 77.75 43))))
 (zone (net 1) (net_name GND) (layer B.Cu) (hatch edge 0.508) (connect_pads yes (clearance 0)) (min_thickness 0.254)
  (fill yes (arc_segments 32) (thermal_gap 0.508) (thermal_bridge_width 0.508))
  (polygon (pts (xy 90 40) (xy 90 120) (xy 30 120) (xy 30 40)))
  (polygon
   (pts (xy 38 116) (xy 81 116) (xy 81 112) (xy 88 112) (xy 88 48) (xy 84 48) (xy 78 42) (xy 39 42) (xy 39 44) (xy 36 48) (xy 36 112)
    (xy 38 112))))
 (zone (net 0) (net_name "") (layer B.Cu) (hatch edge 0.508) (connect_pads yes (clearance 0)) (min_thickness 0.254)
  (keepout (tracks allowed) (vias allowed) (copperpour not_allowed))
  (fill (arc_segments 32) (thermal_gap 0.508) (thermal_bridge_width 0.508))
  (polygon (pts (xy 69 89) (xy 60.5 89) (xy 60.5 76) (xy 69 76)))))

